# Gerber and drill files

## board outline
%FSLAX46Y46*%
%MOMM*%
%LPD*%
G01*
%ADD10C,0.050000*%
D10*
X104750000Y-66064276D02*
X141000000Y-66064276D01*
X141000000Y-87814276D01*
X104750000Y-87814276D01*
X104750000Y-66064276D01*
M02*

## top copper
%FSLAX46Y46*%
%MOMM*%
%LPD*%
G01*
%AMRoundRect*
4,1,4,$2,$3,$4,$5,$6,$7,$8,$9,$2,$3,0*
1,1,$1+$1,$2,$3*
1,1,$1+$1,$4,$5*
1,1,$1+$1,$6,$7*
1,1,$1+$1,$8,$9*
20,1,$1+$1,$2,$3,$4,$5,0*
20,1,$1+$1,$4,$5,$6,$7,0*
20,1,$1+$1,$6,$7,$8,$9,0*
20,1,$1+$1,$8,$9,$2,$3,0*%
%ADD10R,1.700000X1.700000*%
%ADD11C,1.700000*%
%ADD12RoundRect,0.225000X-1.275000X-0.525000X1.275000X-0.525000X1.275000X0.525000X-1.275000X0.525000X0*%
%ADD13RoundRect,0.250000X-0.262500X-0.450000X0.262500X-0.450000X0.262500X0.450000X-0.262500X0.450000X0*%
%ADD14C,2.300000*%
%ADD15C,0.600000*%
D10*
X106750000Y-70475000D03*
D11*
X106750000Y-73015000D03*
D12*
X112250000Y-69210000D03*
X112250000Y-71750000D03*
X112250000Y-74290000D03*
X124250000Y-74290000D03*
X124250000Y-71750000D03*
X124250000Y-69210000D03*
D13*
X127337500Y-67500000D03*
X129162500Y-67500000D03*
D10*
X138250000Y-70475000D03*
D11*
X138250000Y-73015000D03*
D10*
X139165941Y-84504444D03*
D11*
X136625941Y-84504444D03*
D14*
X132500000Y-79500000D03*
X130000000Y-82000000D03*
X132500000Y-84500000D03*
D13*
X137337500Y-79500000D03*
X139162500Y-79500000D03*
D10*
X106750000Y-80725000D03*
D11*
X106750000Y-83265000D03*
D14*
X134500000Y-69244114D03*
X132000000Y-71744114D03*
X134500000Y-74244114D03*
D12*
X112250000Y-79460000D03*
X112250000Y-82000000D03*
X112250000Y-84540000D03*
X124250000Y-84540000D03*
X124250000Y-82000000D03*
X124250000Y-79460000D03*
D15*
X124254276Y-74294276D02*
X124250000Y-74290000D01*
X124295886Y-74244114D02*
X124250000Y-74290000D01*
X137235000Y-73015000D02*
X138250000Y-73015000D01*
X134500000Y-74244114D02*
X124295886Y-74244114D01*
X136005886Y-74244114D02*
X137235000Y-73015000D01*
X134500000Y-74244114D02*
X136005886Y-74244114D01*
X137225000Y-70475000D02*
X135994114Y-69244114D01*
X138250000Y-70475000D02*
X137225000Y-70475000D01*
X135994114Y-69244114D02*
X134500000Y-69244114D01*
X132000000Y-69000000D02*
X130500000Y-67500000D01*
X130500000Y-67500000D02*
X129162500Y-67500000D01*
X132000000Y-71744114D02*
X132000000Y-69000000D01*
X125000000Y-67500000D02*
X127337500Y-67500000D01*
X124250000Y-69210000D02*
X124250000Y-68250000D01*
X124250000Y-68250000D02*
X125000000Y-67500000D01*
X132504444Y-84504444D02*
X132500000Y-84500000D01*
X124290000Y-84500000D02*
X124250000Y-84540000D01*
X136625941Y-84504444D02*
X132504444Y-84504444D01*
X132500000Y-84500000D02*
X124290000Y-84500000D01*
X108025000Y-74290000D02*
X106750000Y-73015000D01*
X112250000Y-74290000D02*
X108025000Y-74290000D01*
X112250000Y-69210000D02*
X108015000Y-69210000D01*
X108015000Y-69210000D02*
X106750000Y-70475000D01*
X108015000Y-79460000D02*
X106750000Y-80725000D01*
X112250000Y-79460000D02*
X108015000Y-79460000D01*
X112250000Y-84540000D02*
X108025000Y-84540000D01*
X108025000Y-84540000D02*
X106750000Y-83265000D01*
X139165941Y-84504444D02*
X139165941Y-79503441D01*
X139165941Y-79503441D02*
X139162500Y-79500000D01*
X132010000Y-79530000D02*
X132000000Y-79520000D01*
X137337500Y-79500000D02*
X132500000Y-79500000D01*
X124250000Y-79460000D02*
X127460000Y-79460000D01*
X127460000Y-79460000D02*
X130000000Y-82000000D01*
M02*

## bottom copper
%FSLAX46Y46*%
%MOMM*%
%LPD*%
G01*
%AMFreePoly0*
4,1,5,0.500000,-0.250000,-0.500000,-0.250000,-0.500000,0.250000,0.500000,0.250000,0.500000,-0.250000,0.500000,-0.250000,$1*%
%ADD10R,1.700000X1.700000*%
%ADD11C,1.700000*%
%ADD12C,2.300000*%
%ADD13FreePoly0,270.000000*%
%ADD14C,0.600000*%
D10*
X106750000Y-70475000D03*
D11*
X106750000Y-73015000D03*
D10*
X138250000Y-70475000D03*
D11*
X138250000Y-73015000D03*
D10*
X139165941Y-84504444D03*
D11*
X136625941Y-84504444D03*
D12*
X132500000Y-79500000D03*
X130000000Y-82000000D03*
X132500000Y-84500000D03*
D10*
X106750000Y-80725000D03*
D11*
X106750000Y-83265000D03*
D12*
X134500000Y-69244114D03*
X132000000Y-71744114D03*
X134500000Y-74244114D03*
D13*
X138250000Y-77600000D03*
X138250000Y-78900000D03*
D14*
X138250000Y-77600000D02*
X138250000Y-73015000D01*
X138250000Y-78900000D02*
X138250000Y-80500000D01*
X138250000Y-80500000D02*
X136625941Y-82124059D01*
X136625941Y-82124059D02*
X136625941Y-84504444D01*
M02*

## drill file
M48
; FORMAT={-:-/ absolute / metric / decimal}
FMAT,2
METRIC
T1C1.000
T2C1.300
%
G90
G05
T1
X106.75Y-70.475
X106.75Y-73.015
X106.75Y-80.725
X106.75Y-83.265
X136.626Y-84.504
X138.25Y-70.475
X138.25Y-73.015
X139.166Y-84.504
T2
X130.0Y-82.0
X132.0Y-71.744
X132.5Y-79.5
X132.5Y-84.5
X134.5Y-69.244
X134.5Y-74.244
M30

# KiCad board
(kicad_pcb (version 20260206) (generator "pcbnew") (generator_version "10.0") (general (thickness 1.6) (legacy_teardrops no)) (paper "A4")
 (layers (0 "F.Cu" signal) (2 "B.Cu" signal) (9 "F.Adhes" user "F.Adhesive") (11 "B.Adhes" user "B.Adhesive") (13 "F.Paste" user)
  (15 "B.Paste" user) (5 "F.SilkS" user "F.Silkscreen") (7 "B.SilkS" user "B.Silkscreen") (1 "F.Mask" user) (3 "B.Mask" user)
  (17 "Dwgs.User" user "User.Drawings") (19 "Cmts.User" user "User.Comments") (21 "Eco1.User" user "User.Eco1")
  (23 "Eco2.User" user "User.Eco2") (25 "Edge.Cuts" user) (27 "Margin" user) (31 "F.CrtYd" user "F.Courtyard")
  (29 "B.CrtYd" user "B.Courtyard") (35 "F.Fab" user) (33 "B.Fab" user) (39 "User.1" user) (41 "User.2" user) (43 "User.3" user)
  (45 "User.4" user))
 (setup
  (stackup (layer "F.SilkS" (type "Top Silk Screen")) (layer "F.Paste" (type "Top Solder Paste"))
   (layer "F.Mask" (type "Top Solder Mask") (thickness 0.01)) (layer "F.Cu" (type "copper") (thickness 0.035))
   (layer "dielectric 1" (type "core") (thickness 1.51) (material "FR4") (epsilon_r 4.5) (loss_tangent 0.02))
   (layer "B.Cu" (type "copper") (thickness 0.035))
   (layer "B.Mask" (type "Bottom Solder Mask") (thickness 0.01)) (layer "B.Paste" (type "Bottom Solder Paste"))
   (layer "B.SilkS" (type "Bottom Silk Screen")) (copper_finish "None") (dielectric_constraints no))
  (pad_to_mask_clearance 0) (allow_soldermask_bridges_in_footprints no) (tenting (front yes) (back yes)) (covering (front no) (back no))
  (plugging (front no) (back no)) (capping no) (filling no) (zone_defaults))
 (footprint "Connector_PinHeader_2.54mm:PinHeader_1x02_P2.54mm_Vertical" (layer "F.Cu") (at 106.75 70.475)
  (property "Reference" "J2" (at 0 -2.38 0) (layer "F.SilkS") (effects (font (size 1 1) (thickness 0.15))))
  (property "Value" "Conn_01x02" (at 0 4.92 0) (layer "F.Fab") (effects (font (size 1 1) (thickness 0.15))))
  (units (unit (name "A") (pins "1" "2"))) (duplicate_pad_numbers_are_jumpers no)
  (pad "1" thru_hole rect (at 0 0) (size 1.7 1.7) (drill 1) (layers "*.Cu" "*.Mask") (remove_unused_layers no) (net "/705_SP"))
  (pad "2" thru_hole circle (at 0 2.54) (size 1.7 1.7) (drill 1) (layers "*.Cu" "*.Mask") (remove_unused_layers no) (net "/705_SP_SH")))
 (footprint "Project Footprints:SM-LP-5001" (layer "F.Cu") (at 118.25 71.75)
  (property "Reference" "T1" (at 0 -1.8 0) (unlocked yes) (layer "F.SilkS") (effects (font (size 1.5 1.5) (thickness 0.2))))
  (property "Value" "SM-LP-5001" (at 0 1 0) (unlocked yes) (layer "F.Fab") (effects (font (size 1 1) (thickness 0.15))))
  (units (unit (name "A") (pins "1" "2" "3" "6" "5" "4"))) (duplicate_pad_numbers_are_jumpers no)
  (pad "1" smd roundrect (at -6 -2.54) (size 3 1.5) (layers "F.Cu" "F.Mask" "F.Paste") (roundrect_rratio 0.15) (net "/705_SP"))
  (pad "2" smd roundrect (at -6 0) (size 3 1.5) (layers "F.Cu" "F.Mask" "F.Paste") (roundrect_rratio 0.15) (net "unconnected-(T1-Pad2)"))
  (pad "3" smd roundrect (at -6 2.54) (size 3 1.5) (layers "F.Cu" "F.Mask" "F.Paste") (roundrect_rratio 0.15) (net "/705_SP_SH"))
  (pad "4" smd roundrect (at 6 2.54) (size 3 1.5) (layers "F.Cu" "F.Mask" "F.Paste") (roundrect_rratio 0.15) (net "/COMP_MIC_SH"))
  (pad "5" smd roundrect (at 6 0) (size 3 1.5) (layers "F.Cu" "F.Mask" "F.Paste") (roundrect_rratio 0.15) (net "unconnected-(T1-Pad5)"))
  (pad "6" smd roundrect (at 6 -2.54) (size 3 1.5) (layers "F.Cu" "F.Mask" "F.Paste") (roundrect_rratio 0.15) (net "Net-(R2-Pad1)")))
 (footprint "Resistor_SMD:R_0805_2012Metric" (layer "F.Cu") (at 128.25 67.5)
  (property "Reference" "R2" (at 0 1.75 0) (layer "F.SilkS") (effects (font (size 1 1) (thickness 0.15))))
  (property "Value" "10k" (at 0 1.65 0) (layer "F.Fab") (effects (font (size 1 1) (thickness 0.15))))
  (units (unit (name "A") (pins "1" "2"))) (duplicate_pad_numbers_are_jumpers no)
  (pad "1" smd roundrect (at -0.9125 0) (size 1.025 1.4) (layers "F.Cu" "F.Mask" "F.Paste") (roundrect_rratio 0.243902)
   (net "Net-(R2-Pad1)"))
  (pad "2" smd roundrect (at 0.9125 0) (size 1.025 1.4) (layers "F.Cu" "F.Mask" "F.Paste") (roundrect_rratio 0.243902) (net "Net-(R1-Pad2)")))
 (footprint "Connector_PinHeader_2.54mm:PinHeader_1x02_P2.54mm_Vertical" (layer "F.Cu") (at 138.25 70.475)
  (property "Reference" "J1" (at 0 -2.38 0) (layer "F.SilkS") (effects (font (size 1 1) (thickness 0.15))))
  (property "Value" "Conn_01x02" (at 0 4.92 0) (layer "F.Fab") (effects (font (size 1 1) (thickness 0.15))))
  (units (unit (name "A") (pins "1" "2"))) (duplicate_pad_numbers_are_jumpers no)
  (pad "1" thru_hole rect (at 0 0) (size 1.7 1.7) (drill 1) (layers "*.Cu" "*.Mask") (remove_unused_layers no) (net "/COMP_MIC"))
  (pad "2" thru_hole circle (at 0 2.54) (size 1.7 1.7) (drill 1) (layers "*.Cu" "*.Mask") (remove_unused_layers no) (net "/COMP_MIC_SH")))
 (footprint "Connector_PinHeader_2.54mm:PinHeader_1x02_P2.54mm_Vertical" (layer "F.Cu") (at 139.165941 84.504444 -90)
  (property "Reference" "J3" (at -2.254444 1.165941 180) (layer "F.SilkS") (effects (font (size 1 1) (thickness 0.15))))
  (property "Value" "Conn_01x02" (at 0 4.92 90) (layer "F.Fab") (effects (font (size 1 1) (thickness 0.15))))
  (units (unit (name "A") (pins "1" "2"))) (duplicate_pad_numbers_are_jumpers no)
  (pad "1" thru_hole rect (at 0 0 270) (size 1.7 1.7) (drill 1) (layers "*.Cu" "*.Mask") (remove_unused_layers no) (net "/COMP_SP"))
  (pad "2" thru_hole circle (at 0 2.54 270) (size 1.7 1.7) (drill 1) (layers "*.Cu" "*.Mask") (remove_unused_layers no) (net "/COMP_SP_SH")))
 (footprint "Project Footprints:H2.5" (layer "F.Cu") (at 131.25 82 -90)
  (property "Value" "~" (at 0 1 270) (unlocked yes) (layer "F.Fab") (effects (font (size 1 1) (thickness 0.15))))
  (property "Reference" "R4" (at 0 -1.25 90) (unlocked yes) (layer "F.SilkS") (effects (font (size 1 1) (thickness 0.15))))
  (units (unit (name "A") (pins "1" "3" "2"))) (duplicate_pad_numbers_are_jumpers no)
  (pad "1" thru_hole circle (at -2.5 -1.25 270) (size 2.3 2.3) (drill 1.3) (layers "*.Cu" "*.Mask") (remove_unused_layers no)
   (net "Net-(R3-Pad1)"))
  (pad "2" thru_hole circle (at 0 1.25 270) (size 2.3 2.3) (drill 1.3) (layers "*.Cu" "*.Mask") (remove_unused_layers no)
   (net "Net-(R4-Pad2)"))
  (pad "3" thru_hole circle (at 2.5 -1.25 270) (size 2.3 2.3) (drill 1.3) (layers "*.Cu" "*.Mask") (remove_unused_layers no)
   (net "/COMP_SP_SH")))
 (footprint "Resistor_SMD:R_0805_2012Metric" (layer "F.Cu") (at 138.25 79.5)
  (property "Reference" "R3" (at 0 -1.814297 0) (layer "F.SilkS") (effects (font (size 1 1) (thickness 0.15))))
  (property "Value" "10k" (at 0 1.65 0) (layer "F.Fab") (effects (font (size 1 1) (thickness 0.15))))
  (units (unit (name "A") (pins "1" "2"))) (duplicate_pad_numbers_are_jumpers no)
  (pad "1" smd roundrect (at -0.9125 0) (size 1.025 1.4) (layers "F.Cu" "F.Mask" "F.Paste") (roundrect_rratio 0.243902)
   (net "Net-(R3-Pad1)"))
  (pad "2" smd roundrect (at 0.9125 0) (size 1.025 1.4) (layers "F.Cu" "F.Mask" "F.Paste") (roundrect_rratio 0.243902) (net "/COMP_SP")))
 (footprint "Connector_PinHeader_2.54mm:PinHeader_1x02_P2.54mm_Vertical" (layer "F.Cu") (at 106.75 80.725)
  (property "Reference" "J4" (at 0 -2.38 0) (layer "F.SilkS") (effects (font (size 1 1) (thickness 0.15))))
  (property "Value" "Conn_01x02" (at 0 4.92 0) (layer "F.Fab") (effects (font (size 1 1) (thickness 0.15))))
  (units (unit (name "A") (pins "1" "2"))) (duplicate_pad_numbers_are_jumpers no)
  (pad "1" thru_hole rect (at 0 0) (size 1.7 1.7) (drill 1) (layers "*.Cu" "*.Mask") (remove_unused_layers no) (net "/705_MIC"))
  (pad "2" thru_hole circle (at 0 2.54) (size 1.7 1.7) (drill 1) (layers "*.Cu" "*.Mask") (remove_unused_layers no) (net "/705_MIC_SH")))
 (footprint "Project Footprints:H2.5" (layer "F.Cu") (at 133.25 71.744114 -90)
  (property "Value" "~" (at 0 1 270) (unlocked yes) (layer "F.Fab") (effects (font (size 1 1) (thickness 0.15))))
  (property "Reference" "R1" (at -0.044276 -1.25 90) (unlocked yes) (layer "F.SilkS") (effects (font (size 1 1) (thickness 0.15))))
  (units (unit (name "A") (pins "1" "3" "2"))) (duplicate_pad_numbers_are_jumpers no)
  (pad "1" thru_hole circle (at -2.5 -1.25 270) (size 2.3 2.3) (drill 1.3) (layers "*.Cu" "*.Mask") (remove_unused_layers no)
   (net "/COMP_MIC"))
  (pad "2" thru_hole circle (at 0 1.25 270) (size 2.3 2.3) (drill 1.3) (layers "*.Cu" "*.Mask") (remove_unused_layers no)
   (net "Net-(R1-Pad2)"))
  (pad "3" thru_hole circle (at 2.5 -1.25 270) (size 2.3 2.3) (drill 1.3) (layers "*.Cu" "*.Mask") (remove_unused_layers no)
   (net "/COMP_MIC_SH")))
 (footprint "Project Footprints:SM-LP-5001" (layer "F.Cu") (at 118.25 82)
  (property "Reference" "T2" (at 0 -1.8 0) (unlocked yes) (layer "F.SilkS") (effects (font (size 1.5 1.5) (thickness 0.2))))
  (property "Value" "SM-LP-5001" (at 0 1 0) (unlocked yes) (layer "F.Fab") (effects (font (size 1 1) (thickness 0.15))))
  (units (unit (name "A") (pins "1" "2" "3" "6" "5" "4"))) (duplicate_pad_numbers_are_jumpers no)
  (pad "1" smd roundrect (at -6 -2.54) (size 3 1.5) (layers "F.Cu" "F.Mask" "F.Paste") (roundrect_rratio 0.15) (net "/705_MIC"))
  (pad "2" smd roundrect (at -6 0) (size 3 1.5) (layers "F.Cu" "F.Mask" "F.Paste") (roundrect_rratio 0.15) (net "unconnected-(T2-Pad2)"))
  (pad "3" smd roundrect (at -6 2.54) (size 3 1.5) (layers "F.Cu" "F.Mask" "F.Paste") (roundrect_rratio 0.15) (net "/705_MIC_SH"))
  (pad "4" smd roundrect (at 6 2.54) (size 3 1.5) (layers "F.Cu" "F.Mask" "F.Paste") (roundrect_rratio 0.15) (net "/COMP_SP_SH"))
  (pad "5" smd roundrect (at 6 0) (size 3 1.5) (layers "F.Cu" "F.Mask" "F.Paste") (roundrect_rratio 0.15) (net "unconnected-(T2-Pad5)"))
  (pad "6" smd roundrect (at 6 -2.54) (size 3 1.5) (layers "F.Cu" "F.Mask" "F.Paste") (roundrect_rratio 0.15) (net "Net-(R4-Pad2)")))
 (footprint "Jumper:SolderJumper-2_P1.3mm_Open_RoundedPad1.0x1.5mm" (layer "B.Cu") (at 138.25 78.25 -90)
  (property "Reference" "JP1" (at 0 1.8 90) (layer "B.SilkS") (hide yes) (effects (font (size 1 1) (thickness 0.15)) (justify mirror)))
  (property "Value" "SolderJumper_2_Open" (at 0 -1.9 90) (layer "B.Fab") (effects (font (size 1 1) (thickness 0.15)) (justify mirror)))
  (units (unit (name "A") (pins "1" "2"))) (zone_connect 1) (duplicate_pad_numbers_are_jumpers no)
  (pad "1" smd custom (at -0.65 0 270) (size 1 0.5) (layers "B.Cu" "B.Mask") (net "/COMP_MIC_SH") (zone_connect 2) (thermal_bridge_angle 45)
   (options (clearance outline) (anchor rect)) (primitives))
  (pad "2" smd custom (at 0.65 0 270) (size 1 0.5) (layers "B.Cu" "B.Mask") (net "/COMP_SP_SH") (zone_connect 2) (thermal_bridge_angle 45)
   (options (clearance outline) (anchor rect)) (primitives)))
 (gr_rect (start 104.75 66.064276) (end 141 87.814276) (stroke (width 0.05) (type default)) (fill no) (layer "Edge.Cuts"))
 (segment (start 124.254276 74.294276) (end 124.25 74.29) (width 0.6) (layer "F.Cu") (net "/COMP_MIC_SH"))
 (segment (start 124.295886 74.244114) (end 124.25 74.29) (width 0.6) (layer "F.Cu") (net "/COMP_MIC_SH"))
 (segment (start 137.235 73.015) (end 138.25 73.015) (width 0.6) (layer "F.Cu") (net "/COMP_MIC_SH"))
 (segment (start 134.5 74.244114) (end 124.295886 74.244114) (width 0.6) (layer "F.Cu") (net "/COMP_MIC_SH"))
 (segment (start 136.005886 74.244114) (end 137.235 73.015) (width 0.6) (layer "F.Cu") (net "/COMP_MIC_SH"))
 (segment (start 134.5 74.244114) (end 136.005886 74.244114) (width 0.6) (layer "F.Cu") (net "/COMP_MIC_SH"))
 (segment (start 138.25 77.6) (end 138.25 73.015) (width 0.6) (layer "B.Cu") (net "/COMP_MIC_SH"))
 (segment (start 137.225 70.475) (end 135.994114 69.244114) (width 0.6) (layer "F.Cu") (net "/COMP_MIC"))
 (segment (start 138.25 70.475) (end 137.225 70.475) (width 0.6) (layer "F.Cu") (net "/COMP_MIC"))
 (segment (start 135.994114 69.244114) (end 134.5 69.244114) (width 0.6) (layer "F.Cu") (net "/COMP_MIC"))
 (segment (start 132 69) (end 130.5 67.5) (width 0.6) (layer "F.Cu") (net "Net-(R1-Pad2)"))
 (segment (start 130.5 67.5) (end 129.1625 67.5) (width 0.6) (layer "F.Cu") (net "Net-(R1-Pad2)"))
 (segment (start 132 71.744114) (end 132 69) (width 0.6) (layer "F.Cu") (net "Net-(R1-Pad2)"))
 (segment (start 125 67.5) (end 127.3375 67.5) (width 0.6) (layer "F.Cu") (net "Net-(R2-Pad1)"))
 (segment (start 124.25 69.21) (end 124.25 68.25) (width 0.6) (layer "F.Cu") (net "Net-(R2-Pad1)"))
 (segment (start 124.25 68.25) (end 125 67.5) (width 0.6) (layer "F.Cu") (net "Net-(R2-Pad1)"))
 (segment (start 132.504444 84.504444) (end 132.5 84.5) (width 0.6) (layer "F.Cu") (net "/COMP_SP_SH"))
 (segment (start 124.29 84.5) (end 124.25 84.54) (width 0.6) (layer "F.Cu") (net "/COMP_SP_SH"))
 (segment (start 136.625941 84.504444) (end 132.504444 84.504444) (width 0.6) (layer "F.Cu") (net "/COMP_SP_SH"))
 (segment (start 132.5 84.5) (end 124.29 84.5) (width 0.6) (layer "F.Cu") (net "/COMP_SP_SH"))
 (segment (start 138.25 78.9) (end 138.25 80.5) (width 0.6) (layer "B.Cu") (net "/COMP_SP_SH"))
 (segment (start 138.25 80.5) (end 136.625941 82.124059) (width 0.6) (layer "B.Cu") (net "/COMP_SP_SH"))
 (segment (start 136.625941 82.124059) (end 136.625941 84.504444) (width 0.6) (layer "B.Cu") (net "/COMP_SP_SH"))
 (segment (start 108.025 74.29) (end 106.75 73.015) (width 0.6) (layer "F.Cu") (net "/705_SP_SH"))
 (segment (start 112.25 74.29) (end 108.025 74.29) (width 0.6) (layer "F.Cu") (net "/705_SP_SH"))
 (segment (start 112.25 69.21) (end 108.015 69.21) (width 0.6) (layer "F.Cu") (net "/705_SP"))
 (segment (start 108.015 69.21) (end 106.75 70.475) (width 0.6) (layer "F.Cu") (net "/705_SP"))
 (segment (start 108.015 79.46) (end 106.75 80.725) (width 0.6) (layer "F.Cu") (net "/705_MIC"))
 (segment (start 112.25 79.46) (end 108.015 79.46) (width 0.6) (layer "F.Cu") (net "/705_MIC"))
 (segment (start 112.25 84.54) (end 108.025 84.54) (width 0.6) (layer "F.Cu") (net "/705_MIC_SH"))
 (segment (start 108.025 84.54) (end 106.75 83.265) (width 0.6) (layer "F.Cu") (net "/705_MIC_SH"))
 (segment (start 139.165941 84.504444) (end 139.165941 79.503441) (width 0.6) (layer "F.Cu") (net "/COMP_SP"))
 (segment (start 139.165941 79.503441) (end 139.1625 79.5) (width 0.6) (layer "F.Cu") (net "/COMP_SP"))
 (segment (start 132.01 79.53) (end 132 79.52) (width 0.6) (layer "F.Cu") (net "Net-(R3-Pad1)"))
 (segment (start 137.3375 79.5) (end 132.5 79.5) (width 0.6) (layer "F.Cu") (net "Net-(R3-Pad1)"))
 (segment (start 124.25 79.46) (end 127.46 79.46) (width 0.6) (layer "F.Cu") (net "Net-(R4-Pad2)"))
 (segment (start 127.46 79.46) (end 130 82) (width 0.6) (layer "F.Cu") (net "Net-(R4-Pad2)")))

